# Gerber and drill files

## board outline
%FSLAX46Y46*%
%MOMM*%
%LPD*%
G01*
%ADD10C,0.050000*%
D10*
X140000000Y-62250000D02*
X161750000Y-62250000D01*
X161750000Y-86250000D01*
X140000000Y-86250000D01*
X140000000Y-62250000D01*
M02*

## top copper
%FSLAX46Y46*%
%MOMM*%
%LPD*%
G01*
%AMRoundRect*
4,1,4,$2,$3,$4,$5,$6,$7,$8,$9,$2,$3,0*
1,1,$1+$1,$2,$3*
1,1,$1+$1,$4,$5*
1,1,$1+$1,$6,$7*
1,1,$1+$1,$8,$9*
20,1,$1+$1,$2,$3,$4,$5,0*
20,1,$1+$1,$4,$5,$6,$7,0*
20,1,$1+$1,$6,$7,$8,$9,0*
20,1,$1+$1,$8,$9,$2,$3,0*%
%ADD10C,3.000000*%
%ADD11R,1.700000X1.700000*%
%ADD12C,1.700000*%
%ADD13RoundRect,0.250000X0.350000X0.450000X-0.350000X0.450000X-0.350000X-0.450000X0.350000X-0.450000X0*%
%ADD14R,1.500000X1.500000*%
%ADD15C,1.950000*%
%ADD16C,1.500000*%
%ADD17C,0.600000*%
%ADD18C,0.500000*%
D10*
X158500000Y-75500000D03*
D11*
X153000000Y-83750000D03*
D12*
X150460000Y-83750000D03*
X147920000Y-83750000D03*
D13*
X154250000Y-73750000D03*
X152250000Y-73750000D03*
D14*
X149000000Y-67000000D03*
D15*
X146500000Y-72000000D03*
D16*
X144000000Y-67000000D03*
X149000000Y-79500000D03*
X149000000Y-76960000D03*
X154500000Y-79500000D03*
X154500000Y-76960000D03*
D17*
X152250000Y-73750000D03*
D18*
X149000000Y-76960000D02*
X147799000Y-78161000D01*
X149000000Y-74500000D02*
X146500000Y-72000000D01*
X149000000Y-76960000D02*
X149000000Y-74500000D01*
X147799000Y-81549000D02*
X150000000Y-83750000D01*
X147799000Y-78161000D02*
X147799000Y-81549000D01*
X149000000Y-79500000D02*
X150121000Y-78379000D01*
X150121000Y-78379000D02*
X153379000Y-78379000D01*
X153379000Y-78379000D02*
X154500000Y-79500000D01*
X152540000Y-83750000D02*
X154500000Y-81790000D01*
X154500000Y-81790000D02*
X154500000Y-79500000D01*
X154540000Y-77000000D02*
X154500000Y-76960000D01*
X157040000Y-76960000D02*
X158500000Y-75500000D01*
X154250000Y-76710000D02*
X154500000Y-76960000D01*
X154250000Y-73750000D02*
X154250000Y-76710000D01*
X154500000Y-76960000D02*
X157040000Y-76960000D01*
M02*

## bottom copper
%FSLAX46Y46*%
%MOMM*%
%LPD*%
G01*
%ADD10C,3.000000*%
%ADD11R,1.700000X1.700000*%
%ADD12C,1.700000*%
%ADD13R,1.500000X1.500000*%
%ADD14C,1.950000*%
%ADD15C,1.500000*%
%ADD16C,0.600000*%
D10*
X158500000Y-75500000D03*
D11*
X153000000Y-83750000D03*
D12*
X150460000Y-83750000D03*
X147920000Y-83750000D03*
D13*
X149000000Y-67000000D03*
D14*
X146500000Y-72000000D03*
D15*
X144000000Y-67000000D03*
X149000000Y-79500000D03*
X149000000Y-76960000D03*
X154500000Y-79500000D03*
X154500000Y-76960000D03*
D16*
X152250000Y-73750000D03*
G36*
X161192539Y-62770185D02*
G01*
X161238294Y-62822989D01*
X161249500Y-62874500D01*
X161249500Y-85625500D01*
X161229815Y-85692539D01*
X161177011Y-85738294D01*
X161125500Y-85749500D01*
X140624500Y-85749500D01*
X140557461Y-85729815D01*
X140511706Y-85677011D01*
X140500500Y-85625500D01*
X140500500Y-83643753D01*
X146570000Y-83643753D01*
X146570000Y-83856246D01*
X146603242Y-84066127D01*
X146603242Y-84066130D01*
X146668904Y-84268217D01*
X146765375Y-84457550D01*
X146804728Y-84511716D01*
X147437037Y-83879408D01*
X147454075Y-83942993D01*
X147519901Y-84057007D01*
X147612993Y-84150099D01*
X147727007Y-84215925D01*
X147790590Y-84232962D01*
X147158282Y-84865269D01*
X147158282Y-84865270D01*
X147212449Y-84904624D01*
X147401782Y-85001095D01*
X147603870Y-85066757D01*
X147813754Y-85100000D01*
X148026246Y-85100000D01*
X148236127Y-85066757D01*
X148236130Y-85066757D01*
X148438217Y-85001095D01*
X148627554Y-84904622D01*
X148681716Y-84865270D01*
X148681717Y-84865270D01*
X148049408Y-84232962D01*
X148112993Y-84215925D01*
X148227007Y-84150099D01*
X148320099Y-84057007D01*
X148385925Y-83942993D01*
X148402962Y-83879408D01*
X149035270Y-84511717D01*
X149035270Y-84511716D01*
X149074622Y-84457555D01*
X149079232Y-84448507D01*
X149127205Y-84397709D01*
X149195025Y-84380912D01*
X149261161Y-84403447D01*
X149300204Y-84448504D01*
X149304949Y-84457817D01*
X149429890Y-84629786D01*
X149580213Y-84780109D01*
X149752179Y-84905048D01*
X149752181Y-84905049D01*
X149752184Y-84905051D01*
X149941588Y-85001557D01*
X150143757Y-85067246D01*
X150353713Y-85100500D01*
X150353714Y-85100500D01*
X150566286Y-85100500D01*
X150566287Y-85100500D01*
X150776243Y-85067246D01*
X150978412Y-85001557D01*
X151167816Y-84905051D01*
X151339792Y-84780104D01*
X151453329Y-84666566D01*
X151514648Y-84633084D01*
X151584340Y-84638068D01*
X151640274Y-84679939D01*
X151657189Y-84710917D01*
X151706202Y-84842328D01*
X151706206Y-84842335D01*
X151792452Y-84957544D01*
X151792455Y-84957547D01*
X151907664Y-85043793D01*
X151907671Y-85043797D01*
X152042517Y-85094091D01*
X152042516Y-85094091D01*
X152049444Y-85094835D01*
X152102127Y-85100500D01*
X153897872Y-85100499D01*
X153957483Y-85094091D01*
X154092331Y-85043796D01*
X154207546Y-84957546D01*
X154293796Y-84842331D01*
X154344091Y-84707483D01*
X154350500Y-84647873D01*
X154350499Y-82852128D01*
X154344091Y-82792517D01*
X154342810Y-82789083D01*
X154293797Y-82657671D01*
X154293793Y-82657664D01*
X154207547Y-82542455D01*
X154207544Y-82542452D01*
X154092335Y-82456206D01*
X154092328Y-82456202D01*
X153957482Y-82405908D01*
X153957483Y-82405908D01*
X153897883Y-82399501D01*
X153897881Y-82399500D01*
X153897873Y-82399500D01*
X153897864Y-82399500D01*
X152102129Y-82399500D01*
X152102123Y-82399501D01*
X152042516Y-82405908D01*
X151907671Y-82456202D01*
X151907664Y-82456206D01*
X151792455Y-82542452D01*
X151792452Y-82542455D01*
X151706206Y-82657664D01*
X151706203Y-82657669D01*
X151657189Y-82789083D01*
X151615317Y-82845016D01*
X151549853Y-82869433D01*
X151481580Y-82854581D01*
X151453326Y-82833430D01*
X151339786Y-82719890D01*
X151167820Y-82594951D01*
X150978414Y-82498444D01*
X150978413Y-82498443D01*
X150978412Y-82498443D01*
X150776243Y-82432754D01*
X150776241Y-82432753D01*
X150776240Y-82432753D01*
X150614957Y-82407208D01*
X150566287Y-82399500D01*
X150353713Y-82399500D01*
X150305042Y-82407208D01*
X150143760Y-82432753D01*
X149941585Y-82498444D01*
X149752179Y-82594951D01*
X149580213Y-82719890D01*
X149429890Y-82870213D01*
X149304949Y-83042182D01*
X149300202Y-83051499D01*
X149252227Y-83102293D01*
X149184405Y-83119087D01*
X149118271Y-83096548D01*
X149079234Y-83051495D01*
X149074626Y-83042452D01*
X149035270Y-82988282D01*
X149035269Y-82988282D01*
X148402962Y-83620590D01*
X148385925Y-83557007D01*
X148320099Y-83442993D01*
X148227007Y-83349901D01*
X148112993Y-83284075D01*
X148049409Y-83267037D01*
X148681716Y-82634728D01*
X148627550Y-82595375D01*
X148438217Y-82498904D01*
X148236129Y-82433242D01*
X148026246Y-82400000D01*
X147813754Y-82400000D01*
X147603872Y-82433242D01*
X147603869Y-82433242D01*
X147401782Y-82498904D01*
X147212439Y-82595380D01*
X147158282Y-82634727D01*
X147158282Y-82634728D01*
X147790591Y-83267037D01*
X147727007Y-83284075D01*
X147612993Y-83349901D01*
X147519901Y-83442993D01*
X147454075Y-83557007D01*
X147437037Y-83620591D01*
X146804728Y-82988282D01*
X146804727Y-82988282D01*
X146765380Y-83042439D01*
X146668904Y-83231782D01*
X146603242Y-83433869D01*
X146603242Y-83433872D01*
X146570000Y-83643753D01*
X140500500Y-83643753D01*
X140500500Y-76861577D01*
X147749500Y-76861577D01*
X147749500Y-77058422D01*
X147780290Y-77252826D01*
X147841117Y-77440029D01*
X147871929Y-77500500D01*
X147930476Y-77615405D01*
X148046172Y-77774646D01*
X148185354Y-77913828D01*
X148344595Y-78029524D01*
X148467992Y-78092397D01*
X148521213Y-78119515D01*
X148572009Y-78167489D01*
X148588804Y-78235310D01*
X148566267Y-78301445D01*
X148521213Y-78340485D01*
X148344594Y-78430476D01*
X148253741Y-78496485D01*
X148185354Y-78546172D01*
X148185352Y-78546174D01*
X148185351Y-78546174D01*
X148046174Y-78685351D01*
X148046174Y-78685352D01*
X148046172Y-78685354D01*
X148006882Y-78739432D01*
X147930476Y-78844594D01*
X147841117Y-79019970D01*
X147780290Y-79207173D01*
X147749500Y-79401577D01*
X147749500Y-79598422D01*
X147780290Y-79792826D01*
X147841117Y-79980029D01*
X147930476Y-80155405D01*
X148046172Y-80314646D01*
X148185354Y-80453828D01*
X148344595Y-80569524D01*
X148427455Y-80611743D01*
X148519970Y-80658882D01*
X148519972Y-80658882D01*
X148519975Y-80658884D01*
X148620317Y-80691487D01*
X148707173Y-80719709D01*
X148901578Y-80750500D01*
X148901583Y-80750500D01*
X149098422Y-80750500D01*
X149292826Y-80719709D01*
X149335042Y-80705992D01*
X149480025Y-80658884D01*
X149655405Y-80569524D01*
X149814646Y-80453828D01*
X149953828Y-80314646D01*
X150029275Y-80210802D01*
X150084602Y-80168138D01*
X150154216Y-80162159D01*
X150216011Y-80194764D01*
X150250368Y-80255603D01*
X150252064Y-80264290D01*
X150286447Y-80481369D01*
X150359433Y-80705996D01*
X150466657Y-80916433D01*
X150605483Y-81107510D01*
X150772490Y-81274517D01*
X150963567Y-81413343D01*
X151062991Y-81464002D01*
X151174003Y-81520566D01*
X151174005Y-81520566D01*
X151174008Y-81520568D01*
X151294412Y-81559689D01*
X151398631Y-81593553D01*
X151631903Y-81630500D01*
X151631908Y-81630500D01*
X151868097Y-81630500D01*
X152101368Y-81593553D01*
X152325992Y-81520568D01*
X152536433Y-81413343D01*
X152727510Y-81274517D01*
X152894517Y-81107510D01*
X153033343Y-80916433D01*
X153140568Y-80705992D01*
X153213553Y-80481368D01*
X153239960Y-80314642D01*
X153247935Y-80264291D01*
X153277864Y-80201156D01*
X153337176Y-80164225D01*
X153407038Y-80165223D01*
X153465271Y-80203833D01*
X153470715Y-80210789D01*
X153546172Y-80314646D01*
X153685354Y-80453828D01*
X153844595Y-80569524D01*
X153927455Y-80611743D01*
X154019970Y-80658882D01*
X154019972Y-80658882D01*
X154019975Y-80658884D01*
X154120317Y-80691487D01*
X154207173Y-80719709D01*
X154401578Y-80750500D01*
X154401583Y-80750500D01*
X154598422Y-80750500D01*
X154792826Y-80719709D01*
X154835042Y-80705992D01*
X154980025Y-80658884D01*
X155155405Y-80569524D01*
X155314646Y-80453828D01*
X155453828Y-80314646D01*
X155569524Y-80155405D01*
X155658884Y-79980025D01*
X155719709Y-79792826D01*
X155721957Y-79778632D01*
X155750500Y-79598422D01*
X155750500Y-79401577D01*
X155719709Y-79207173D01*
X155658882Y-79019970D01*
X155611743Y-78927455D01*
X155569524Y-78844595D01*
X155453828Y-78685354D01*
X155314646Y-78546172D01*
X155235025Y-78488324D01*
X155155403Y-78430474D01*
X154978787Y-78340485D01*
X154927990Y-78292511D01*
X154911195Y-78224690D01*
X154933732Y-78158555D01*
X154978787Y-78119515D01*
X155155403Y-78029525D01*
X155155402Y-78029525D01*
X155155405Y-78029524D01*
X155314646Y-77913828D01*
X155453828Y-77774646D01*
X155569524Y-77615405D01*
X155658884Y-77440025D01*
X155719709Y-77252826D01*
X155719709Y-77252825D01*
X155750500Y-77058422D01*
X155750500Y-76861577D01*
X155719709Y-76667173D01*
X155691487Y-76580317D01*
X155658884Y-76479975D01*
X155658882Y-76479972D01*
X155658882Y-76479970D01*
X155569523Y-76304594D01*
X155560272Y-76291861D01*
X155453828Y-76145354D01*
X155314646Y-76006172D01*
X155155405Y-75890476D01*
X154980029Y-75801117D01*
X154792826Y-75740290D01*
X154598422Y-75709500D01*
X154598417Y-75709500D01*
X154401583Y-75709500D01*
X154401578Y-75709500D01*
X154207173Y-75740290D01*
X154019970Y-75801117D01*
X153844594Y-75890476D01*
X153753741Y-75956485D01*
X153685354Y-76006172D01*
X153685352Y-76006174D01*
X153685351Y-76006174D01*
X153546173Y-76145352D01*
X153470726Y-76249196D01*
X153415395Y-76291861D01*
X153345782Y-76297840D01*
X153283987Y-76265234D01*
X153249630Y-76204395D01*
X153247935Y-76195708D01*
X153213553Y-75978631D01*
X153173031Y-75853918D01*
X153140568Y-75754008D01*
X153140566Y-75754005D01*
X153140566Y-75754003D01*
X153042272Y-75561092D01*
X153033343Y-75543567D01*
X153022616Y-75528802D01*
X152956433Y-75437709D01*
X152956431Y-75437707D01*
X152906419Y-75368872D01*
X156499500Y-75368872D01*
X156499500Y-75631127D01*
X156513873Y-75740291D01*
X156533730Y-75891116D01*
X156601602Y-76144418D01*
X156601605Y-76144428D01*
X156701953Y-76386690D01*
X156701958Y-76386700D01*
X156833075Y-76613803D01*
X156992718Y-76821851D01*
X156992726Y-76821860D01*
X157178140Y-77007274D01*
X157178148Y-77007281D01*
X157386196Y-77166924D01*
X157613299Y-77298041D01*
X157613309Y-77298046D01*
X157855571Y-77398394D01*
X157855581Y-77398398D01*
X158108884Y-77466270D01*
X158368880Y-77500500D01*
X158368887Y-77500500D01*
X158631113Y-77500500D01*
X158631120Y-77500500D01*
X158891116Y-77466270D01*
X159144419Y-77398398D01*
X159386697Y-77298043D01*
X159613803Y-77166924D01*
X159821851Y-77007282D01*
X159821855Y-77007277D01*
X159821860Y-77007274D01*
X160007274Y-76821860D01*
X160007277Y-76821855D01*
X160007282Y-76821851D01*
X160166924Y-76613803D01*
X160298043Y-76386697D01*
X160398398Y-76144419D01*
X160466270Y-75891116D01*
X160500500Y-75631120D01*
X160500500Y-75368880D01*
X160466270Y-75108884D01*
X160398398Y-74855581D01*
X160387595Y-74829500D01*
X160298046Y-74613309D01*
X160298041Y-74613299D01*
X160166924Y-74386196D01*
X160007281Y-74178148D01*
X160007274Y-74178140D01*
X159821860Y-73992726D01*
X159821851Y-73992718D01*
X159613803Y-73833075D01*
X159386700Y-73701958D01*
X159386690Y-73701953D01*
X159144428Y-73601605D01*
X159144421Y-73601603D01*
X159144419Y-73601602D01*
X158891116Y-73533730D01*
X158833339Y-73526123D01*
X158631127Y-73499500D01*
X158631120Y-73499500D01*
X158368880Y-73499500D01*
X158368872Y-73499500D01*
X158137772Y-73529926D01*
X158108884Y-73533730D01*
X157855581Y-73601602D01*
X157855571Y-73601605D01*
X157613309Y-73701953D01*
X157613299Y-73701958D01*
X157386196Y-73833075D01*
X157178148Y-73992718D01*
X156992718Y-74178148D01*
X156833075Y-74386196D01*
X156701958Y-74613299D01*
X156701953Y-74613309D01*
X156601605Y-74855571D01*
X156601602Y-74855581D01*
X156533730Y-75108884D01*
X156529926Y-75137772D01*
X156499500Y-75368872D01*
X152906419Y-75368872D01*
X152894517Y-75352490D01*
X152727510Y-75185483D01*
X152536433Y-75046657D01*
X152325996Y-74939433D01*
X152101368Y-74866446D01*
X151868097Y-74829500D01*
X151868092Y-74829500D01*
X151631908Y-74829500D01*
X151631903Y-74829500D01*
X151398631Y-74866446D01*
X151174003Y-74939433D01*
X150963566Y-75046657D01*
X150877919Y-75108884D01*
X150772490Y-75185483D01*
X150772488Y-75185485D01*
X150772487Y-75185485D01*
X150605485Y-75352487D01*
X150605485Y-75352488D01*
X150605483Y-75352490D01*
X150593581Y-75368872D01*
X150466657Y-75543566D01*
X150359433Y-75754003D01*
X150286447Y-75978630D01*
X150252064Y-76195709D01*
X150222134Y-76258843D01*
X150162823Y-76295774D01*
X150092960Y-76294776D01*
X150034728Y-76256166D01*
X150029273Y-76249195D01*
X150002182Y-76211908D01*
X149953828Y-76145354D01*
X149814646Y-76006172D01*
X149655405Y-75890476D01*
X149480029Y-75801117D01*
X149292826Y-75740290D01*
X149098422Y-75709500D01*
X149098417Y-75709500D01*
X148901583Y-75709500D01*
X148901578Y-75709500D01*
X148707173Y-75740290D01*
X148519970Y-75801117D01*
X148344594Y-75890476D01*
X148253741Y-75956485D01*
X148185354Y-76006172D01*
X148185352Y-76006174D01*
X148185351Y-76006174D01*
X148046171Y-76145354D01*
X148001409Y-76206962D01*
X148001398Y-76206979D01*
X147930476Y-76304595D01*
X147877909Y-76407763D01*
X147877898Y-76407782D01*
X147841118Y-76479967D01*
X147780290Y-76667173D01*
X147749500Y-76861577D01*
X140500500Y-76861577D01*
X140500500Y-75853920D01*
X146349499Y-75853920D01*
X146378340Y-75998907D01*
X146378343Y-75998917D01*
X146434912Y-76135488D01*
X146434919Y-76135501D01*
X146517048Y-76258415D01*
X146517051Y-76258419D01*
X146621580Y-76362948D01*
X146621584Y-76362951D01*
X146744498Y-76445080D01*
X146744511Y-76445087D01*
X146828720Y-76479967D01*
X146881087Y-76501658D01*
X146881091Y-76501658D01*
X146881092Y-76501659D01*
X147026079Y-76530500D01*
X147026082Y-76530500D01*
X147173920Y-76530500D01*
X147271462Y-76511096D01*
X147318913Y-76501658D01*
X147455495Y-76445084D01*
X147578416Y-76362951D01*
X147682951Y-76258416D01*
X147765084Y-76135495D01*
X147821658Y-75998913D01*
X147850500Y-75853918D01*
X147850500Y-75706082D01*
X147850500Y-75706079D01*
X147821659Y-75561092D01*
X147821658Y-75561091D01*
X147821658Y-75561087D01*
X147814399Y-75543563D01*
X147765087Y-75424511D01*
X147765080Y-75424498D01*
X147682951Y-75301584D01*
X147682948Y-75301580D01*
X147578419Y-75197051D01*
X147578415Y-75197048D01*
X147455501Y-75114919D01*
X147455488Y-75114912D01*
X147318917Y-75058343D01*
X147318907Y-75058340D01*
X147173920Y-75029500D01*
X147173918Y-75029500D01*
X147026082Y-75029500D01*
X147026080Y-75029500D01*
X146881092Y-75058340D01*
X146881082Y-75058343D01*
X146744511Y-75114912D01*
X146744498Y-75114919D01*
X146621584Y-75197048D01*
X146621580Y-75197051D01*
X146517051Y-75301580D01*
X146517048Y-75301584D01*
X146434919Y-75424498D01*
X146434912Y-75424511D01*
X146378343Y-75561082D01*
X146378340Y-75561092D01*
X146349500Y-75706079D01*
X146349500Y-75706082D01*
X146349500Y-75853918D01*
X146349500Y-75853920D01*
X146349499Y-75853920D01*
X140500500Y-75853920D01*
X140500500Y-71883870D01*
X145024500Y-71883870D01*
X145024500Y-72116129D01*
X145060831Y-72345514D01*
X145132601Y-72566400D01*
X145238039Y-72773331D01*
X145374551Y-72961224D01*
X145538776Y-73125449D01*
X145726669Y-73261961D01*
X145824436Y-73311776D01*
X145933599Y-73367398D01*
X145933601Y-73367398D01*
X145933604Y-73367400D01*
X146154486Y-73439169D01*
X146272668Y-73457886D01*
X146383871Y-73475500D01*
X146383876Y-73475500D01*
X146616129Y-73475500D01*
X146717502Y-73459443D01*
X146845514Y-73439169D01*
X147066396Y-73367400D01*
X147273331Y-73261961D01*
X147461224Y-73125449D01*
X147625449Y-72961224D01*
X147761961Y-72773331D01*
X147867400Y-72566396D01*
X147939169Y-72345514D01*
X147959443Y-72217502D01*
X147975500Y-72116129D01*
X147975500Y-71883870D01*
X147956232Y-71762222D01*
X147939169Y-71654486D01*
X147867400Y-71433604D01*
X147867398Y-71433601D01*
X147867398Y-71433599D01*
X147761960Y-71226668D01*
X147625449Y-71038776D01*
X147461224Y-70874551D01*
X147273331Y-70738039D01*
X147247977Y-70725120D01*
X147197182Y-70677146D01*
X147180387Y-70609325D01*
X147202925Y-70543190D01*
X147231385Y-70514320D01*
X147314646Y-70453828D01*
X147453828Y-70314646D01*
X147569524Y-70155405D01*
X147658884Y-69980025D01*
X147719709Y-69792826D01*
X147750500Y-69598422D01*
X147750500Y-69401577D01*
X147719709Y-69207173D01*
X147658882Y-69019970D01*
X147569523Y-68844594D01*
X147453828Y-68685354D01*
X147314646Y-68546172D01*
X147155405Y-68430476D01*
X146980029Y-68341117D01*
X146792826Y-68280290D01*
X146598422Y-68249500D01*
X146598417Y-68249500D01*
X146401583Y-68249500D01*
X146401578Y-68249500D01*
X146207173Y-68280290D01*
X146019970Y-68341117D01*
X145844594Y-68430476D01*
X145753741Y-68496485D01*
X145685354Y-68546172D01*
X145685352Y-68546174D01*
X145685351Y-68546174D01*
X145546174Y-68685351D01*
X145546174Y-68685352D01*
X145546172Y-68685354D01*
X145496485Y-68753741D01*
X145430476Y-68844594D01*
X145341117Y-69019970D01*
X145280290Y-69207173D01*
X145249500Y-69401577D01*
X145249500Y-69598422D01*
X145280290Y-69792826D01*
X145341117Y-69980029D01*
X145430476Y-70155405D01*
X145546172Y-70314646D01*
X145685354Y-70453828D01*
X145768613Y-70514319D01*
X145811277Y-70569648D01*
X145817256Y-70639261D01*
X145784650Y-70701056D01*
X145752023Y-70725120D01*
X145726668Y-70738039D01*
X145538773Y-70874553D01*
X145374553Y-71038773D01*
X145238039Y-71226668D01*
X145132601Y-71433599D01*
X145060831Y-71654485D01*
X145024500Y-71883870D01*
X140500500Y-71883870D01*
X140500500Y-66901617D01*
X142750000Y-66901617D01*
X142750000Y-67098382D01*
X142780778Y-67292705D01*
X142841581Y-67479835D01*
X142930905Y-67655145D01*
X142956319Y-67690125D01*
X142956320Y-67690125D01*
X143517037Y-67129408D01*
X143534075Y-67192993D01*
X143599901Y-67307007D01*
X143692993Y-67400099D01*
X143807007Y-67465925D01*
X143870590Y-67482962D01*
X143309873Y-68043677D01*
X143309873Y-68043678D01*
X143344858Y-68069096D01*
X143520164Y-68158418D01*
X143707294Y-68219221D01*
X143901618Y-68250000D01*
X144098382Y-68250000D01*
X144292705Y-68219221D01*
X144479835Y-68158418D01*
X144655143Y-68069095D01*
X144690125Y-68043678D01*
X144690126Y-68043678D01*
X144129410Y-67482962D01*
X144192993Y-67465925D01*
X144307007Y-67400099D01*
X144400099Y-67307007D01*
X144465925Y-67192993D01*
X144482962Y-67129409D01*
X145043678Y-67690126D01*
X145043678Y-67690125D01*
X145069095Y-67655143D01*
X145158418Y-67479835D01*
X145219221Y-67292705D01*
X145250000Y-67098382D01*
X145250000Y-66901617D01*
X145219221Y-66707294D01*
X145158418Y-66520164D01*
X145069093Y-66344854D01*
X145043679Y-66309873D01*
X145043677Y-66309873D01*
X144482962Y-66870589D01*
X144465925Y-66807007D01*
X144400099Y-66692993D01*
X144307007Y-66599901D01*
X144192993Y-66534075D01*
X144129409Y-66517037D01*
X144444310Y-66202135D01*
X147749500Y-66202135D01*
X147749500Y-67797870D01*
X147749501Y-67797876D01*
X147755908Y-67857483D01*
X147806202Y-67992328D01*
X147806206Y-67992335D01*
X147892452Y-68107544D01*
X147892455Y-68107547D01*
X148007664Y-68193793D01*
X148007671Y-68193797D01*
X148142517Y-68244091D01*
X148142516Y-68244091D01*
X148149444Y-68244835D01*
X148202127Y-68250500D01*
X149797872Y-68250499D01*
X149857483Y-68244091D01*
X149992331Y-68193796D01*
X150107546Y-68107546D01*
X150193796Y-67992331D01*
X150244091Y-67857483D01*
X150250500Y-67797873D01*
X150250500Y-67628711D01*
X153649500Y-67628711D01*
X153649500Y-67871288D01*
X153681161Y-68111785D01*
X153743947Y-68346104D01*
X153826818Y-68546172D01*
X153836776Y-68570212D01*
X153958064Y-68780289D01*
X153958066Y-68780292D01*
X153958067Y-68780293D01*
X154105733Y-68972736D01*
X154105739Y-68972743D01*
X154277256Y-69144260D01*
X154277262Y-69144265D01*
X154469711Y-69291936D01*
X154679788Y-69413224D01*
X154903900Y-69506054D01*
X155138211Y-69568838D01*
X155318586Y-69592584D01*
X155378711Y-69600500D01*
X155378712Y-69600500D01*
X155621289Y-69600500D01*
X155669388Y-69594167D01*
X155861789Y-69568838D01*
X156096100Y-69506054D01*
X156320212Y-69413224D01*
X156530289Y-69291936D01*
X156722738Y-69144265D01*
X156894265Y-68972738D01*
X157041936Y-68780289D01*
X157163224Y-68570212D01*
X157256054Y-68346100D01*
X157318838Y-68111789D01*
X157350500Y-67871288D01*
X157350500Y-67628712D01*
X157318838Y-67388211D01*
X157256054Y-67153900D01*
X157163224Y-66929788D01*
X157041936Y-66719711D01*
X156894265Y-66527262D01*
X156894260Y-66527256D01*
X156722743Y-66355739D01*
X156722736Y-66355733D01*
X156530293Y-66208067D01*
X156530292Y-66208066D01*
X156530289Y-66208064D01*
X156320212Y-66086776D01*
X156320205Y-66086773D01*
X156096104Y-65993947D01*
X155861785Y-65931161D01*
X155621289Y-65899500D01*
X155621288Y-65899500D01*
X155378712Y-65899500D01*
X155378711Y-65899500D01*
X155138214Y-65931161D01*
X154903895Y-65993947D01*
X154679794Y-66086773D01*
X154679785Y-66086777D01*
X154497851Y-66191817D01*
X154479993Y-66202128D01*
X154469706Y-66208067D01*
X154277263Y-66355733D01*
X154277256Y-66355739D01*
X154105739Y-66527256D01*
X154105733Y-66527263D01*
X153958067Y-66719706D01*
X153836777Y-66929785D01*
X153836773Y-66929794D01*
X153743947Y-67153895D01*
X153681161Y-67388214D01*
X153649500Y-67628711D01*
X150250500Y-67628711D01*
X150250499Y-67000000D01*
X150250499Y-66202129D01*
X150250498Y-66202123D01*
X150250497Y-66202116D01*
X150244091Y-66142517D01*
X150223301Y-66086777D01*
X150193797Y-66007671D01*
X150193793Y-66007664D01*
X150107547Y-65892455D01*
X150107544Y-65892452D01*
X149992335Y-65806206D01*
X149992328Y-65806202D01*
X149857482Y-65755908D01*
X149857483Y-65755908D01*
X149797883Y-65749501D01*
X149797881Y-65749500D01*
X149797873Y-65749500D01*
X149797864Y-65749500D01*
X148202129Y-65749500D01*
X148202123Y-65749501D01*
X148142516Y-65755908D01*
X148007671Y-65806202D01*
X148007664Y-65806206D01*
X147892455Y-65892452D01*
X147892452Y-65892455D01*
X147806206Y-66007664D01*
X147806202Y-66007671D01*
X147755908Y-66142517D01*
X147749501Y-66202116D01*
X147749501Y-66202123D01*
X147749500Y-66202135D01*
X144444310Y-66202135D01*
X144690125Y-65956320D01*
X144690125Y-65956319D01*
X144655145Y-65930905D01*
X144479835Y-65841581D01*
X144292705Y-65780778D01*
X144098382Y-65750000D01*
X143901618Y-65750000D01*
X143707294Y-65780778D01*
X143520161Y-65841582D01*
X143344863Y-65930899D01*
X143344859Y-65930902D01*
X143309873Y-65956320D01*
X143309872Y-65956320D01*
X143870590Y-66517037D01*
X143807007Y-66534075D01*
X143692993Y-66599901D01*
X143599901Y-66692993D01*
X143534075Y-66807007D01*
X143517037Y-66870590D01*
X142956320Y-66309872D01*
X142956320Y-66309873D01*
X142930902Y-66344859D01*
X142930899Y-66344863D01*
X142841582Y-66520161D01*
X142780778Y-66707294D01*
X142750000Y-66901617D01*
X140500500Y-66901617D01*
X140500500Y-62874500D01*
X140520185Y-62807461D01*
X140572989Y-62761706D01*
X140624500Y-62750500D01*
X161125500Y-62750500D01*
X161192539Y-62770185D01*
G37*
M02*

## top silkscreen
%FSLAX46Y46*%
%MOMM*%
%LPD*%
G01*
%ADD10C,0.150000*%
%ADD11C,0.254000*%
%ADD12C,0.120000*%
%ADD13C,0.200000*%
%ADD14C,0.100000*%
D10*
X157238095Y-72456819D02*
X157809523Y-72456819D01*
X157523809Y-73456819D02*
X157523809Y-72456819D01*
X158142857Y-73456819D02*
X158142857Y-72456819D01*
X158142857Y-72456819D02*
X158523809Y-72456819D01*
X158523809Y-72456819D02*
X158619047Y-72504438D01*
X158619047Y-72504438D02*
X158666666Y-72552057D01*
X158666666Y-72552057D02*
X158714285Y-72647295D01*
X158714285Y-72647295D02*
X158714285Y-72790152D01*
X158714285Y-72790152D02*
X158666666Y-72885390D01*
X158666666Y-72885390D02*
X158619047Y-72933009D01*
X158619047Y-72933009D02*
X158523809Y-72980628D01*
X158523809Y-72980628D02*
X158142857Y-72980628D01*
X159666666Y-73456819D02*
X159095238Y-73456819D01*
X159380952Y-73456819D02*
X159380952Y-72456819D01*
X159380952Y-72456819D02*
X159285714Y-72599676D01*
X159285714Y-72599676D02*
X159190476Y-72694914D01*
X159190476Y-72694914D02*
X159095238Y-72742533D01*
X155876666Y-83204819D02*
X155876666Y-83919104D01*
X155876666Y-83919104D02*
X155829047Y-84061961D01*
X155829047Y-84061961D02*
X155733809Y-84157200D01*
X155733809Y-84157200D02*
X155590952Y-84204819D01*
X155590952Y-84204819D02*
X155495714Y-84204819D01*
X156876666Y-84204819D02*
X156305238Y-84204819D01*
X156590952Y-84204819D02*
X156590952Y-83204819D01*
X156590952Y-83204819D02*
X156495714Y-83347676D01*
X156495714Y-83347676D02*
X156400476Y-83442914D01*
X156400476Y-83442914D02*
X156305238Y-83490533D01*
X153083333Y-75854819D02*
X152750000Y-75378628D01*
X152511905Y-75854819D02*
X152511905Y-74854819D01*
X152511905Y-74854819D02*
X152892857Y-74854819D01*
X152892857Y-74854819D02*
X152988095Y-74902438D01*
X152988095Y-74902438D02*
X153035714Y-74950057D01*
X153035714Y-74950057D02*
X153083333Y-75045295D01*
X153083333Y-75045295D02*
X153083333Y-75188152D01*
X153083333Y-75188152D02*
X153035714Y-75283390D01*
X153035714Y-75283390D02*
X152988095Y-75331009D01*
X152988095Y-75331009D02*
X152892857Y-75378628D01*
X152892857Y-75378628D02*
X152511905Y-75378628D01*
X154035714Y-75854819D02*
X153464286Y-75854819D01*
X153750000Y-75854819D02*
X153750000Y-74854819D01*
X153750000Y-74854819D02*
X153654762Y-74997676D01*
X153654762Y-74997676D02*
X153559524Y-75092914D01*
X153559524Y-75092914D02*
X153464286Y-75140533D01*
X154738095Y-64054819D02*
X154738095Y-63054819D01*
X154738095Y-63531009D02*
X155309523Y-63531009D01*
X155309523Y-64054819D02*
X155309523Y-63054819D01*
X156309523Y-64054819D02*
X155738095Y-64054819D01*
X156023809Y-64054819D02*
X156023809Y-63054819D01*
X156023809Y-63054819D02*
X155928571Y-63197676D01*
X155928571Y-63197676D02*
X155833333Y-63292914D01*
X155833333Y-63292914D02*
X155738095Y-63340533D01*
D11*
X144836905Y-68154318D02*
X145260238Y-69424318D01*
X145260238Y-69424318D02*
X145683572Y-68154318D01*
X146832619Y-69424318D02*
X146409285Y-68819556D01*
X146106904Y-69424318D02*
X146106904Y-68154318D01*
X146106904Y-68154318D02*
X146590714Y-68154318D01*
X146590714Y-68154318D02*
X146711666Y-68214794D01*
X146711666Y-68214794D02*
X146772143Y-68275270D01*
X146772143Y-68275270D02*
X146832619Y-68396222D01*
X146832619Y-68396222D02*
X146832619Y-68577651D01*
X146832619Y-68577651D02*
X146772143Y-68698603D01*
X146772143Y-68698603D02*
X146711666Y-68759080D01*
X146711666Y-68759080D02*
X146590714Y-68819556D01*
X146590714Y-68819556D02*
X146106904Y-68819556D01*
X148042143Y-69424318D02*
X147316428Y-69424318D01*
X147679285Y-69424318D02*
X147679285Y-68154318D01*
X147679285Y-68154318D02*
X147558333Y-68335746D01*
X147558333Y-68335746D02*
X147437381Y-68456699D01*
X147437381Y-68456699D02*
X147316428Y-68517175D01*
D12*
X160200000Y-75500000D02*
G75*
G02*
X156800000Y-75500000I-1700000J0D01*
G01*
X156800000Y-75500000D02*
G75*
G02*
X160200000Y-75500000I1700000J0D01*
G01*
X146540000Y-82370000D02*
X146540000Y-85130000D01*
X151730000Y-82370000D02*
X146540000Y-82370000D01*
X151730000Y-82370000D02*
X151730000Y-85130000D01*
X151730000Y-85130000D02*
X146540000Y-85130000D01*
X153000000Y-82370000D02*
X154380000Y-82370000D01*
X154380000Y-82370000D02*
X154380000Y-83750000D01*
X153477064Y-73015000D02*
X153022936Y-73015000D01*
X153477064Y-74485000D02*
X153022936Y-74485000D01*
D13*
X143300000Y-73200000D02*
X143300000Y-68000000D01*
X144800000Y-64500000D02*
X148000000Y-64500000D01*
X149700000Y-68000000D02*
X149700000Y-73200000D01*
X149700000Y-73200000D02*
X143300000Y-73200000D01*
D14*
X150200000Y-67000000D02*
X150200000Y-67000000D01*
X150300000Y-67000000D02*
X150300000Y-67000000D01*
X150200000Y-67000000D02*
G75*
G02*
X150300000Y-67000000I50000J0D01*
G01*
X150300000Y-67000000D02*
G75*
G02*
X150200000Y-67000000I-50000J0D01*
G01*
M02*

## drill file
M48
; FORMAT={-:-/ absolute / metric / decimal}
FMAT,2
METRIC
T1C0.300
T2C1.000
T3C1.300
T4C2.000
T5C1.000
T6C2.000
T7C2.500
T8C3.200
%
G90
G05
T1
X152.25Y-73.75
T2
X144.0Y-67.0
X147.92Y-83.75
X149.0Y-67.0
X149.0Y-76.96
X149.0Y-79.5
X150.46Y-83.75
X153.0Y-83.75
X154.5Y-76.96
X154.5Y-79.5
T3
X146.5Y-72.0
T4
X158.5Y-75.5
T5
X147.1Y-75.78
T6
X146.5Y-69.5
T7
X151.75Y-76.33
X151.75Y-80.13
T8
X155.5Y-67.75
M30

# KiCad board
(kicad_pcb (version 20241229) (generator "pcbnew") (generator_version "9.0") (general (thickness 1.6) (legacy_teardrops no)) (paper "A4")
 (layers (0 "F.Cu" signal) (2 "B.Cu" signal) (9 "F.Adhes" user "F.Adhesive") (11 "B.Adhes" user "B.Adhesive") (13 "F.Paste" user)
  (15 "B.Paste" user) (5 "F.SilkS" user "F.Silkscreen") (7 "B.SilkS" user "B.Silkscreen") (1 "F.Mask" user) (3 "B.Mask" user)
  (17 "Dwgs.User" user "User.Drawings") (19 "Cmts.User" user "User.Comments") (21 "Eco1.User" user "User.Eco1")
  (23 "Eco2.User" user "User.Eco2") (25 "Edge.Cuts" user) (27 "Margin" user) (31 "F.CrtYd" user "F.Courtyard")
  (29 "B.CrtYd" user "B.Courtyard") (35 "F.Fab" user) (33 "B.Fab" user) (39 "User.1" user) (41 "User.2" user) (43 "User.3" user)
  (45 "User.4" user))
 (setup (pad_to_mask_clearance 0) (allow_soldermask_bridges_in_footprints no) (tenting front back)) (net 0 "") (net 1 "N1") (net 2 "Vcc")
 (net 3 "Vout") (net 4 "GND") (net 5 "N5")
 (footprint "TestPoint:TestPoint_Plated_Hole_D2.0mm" (layer "F.Cu") (at 158.5 75.5)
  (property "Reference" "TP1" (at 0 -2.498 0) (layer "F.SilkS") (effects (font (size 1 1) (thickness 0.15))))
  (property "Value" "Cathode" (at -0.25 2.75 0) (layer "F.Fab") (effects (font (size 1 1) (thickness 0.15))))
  (fp_circle (center 0 0) (end 0 -1.7) (stroke (width 0.12) (type solid)) (fill no) (layer "F.SilkS"))
  (pad "1" thru_hole circle (at 0 0) (size 3 3) (drill 2) (layers "*.Cu" "*.Mask") (remove_unused_layers no) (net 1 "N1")))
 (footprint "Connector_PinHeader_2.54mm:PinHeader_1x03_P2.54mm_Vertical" (layer "F.Cu") (at 153 83.75 -90)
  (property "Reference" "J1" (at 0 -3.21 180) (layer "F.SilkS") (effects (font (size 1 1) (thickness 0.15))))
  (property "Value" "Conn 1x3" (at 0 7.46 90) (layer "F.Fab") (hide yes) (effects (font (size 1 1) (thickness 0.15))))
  (fp_line (start -1.38 6.46) (end 1.38 6.46) (stroke (width 0.12) (type solid)) (layer "F.SilkS"))
  (fp_line (start -1.38 1.27) (end -1.38 6.46) (stroke (width 0.12) (type solid)) (layer "F.SilkS"))
  (fp_line (start -1.38 1.27) (end 1.38 1.27) (stroke (width 0.12) (type solid)) (layer "F.SilkS"))
  (fp_line (start 1.38 1.27) (end 1.38 6.46) (stroke (width 0.12) (type solid)) (layer "F.SilkS"))
  (fp_line (start -1.38 0) (end -1.38 -1.38) (stroke (width 0.12) (type solid)) (layer "F.SilkS"))
  (fp_line (start -1.38 -1.38) (end 0 -1.38) (stroke (width 0.12) (type solid)) (layer "F.SilkS"))
  (pad "1" thru_hole rect (at 0 0 270) (size 1.7 1.7) (drill 1) (layers "*.Cu" "*.Mask") (remove_unused_layers no) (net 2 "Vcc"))
  (pad "2" thru_hole circle (at 0 2.54 270) (size 1.7 1.7) (drill 1) (layers "*.Cu" "*.Mask") (remove_unused_layers no) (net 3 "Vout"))
  (pad "3" thru_hole circle (at 0 5.08 270) (size 1.7 1.7) (drill 1) (layers "*.Cu" "*.Mask") (remove_unused_layers no) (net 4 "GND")))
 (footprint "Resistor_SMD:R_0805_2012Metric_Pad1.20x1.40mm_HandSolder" (layer "F.Cu") (at 153.25 73.75 180)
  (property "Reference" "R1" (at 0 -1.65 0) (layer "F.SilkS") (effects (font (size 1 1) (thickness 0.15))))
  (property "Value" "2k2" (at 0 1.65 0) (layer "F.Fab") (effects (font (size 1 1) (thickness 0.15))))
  (fp_line (start -0.227064 0.735) (end 0.227064 0.735) (stroke (width 0.12) (type solid)) (layer "F.SilkS"))
  (fp_line (start -0.227064 -0.735) (end 0.227064 -0.735) (stroke (width 0.12) (type solid)) (layer "F.SilkS"))
  (pad "1" smd roundrect (at -1 0 180) (size 1.2 1.4) (layers "F.Cu" "F.Mask" "F.Paste") (roundrect_rratio 0.208333) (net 1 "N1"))
  (pad "2" smd roundrect (at 1 0 180) (size 1.2 1.4) (layers "F.Cu" "F.Mask" "F.Paste") (roundrect_rratio 0.208333) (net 4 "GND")))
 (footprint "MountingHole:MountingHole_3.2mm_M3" (layer "F.Cu") (at 155.5 67.75)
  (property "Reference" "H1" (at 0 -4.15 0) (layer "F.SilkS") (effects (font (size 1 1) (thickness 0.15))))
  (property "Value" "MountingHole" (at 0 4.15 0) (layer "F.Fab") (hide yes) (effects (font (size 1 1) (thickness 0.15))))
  (pad "" np_thru_hole circle (at 0 0) (size 3.2 3.2) (drill 3.2) (layers "*.Cu" "*.Mask")))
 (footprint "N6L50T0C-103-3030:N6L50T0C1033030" (layer "F.Cu") (at 149 67 180)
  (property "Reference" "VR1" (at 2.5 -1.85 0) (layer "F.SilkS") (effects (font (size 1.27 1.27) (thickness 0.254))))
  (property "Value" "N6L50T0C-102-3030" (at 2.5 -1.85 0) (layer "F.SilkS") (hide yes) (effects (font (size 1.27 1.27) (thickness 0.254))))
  (fp_line (start 5.7 -6.2) (end 5.7 -1) (stroke (width 0.2) (type solid)) (layer "F.SilkS"))
  (fp_line (start 4.2 2.5) (end 1 2.5) (stroke (width 0.2) (type solid)) (layer "F.SilkS"))
  (fp_line (start -0.7 -1) (end -0.7 -6.2) (stroke (width 0.2) (type solid)) (layer "F.SilkS"))
  (fp_line (start -0.7 -6.2) (end 5.7 -6.2) (stroke (width 0.2) (type solid)) (layer "F.SilkS"))
  (fp_line (start -1.2 0) (end -1.2 0) (stroke (width 0.1) (type solid)) (layer "F.SilkS"))
  (fp_line (start -1.3 0) (end -1.3 0) (stroke (width 0.1) (type solid)) (layer "F.SilkS"))
  (fp_arc (start -1.2 0) (mid -1.25 0.05) (end -1.3 0) (stroke (width 0.1) (type solid)) (layer "F.SilkS"))
  (fp_arc (start -1.3 0) (mid -1.25 -0.05) (end -1.2 0) (stroke (width 0.1) (type solid)) (layer "F.SilkS"))
  (pad "" np_thru_hole circle (at 2.5 -2.5 180) (size 2 2) (drill 2) (layers "*.Cu" "*.Mask"))
  (pad "1" thru_hole rect (at 0 0 180) (size 1.5 1.5) (drill 1) (layers "*.Cu" "*.Mask") (remove_unused_layers no) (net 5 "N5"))
  (pad "2" thru_hole circle (at 2.5 -5 180) (size 1.95 1.95) (drill 1.3) (layers "*.Cu" "*.Mask") (remove_unused_layers no) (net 3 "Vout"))
  (pad "3" thru_hole circle (at 5 0 180) (size 1.5 1.5) (drill 1) (layers "*.Cu" "*.Mask") (remove_unused_layers no) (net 4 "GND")))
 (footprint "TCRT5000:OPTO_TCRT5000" (layer "B.Cu") (at 151.75 78.23)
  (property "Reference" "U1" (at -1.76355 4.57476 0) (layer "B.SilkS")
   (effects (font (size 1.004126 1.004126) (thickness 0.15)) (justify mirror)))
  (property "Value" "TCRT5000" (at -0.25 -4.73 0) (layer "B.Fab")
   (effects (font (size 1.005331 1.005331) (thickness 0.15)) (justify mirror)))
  (pad "" np_thru_hole circle (at -4.65 -2.45) (size 1 1) (drill 1) (layers "*.Cu" "*.Mask"))
  (pad "" np_thru_hole circle (at 0 -1.9) (size 2.5 2.5) (drill 2.5) (layers "*.Cu" "*.Mask"))
  (pad "" np_thru_hole circle (at 0 1.9) (size 2.5 2.5) (drill 2.5) (layers "*.Cu" "*.Mask"))
  (pad "1" thru_hole circle (at -2.75 1.27) (size 1.5 1.5) (drill 1) (layers "*.Cu" "*.Mask") (remove_unused_layers no) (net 2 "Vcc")
   (solder_mask_margin 0.102))
  (pad "2" thru_hole circle (at -2.75 -1.27) (size 1.5 1.5) (drill 1) (layers "*.Cu" "*.Mask") (remove_unused_layers no) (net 3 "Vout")
   (solder_mask_margin 0.102))
  (pad "3" thru_hole circle (at 2.75 1.27) (size 1.5 1.5) (drill 1) (layers "*.Cu" "*.Mask") (remove_unused_layers no) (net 2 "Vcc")
   (solder_mask_margin 0.102))
  (pad "4" thru_hole circle (at 2.75 -1.27) (size 1.5 1.5) (drill 1) (layers "*.Cu" "*.Mask") (remove_unused_layers no) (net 1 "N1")
   (solder_mask_margin 0.102)))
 (gr_rect (start 140 62.25) (end 161.75 86.25) (stroke (width 0.05) (type default)) (fill no) (layer "Edge.Cuts"))
 (segment (start 149 76.96) (end 147.799 78.161) (width 0.5) (layer "F.Cu") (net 3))
 (segment (start 149 74.5) (end 146.5 72) (width 0.5) (layer "F.Cu") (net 3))
 (segment (start 149 76.96) (end 149 74.5) (width 0.5) (layer "F.Cu") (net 3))
 (segment (start 147.799 81.549) (end 150 83.75) (width 0.5) (layer "F.Cu") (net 3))
 (segment (start 147.799 78.161) (end 147.799 81.549) (width 0.5) (layer "F.Cu") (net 3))
 (via (at 152.25 73.75) (size 0.6) (drill 0.3) (layers "F.Cu" "B.Cu") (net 4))
 (segment (start 149 79.5) (end 150.121 78.379) (width 0.5) (layer "F.Cu") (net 2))
 (segment (start 150.121 78.379) (end 153.379 78.379) (width 0.5) (layer "F.Cu") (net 2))
 (segment (start 153.379 78.379) (end 154.5 79.5) (width 0.5) (layer "F.Cu") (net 2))
 (segment (start 152.54 83.75) (end 154.5 81.79) (width 0.5) (layer "F.Cu") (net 2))
 (segment (start 154.5 81.79) (end 154.5 79.5) (width 0.5) (layer "F.Cu") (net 2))
 (segment (start 154.54 77) (end 154.5 76.96) (width 0.5) (layer "F.Cu") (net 1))
 (segment (start 157.04 76.96) (end 158.5 75.5) (width 0.5) (layer "F.Cu") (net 1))
 (segment (start 154.25 76.71) (end 154.5 76.96) (width 0.5) (layer "F.Cu") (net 1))
 (segment (start 154.25 73.75) (end 154.25 76.71) (width 0.5) (layer "F.Cu") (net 1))
 (segment (start 154.5 76.96) (end 157.04 76.96) (width 0.5) (layer "F.Cu") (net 1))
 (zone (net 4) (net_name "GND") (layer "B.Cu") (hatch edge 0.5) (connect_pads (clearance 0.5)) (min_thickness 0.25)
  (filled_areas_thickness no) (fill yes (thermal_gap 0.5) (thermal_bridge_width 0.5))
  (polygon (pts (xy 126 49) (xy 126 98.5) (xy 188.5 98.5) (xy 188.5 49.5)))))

